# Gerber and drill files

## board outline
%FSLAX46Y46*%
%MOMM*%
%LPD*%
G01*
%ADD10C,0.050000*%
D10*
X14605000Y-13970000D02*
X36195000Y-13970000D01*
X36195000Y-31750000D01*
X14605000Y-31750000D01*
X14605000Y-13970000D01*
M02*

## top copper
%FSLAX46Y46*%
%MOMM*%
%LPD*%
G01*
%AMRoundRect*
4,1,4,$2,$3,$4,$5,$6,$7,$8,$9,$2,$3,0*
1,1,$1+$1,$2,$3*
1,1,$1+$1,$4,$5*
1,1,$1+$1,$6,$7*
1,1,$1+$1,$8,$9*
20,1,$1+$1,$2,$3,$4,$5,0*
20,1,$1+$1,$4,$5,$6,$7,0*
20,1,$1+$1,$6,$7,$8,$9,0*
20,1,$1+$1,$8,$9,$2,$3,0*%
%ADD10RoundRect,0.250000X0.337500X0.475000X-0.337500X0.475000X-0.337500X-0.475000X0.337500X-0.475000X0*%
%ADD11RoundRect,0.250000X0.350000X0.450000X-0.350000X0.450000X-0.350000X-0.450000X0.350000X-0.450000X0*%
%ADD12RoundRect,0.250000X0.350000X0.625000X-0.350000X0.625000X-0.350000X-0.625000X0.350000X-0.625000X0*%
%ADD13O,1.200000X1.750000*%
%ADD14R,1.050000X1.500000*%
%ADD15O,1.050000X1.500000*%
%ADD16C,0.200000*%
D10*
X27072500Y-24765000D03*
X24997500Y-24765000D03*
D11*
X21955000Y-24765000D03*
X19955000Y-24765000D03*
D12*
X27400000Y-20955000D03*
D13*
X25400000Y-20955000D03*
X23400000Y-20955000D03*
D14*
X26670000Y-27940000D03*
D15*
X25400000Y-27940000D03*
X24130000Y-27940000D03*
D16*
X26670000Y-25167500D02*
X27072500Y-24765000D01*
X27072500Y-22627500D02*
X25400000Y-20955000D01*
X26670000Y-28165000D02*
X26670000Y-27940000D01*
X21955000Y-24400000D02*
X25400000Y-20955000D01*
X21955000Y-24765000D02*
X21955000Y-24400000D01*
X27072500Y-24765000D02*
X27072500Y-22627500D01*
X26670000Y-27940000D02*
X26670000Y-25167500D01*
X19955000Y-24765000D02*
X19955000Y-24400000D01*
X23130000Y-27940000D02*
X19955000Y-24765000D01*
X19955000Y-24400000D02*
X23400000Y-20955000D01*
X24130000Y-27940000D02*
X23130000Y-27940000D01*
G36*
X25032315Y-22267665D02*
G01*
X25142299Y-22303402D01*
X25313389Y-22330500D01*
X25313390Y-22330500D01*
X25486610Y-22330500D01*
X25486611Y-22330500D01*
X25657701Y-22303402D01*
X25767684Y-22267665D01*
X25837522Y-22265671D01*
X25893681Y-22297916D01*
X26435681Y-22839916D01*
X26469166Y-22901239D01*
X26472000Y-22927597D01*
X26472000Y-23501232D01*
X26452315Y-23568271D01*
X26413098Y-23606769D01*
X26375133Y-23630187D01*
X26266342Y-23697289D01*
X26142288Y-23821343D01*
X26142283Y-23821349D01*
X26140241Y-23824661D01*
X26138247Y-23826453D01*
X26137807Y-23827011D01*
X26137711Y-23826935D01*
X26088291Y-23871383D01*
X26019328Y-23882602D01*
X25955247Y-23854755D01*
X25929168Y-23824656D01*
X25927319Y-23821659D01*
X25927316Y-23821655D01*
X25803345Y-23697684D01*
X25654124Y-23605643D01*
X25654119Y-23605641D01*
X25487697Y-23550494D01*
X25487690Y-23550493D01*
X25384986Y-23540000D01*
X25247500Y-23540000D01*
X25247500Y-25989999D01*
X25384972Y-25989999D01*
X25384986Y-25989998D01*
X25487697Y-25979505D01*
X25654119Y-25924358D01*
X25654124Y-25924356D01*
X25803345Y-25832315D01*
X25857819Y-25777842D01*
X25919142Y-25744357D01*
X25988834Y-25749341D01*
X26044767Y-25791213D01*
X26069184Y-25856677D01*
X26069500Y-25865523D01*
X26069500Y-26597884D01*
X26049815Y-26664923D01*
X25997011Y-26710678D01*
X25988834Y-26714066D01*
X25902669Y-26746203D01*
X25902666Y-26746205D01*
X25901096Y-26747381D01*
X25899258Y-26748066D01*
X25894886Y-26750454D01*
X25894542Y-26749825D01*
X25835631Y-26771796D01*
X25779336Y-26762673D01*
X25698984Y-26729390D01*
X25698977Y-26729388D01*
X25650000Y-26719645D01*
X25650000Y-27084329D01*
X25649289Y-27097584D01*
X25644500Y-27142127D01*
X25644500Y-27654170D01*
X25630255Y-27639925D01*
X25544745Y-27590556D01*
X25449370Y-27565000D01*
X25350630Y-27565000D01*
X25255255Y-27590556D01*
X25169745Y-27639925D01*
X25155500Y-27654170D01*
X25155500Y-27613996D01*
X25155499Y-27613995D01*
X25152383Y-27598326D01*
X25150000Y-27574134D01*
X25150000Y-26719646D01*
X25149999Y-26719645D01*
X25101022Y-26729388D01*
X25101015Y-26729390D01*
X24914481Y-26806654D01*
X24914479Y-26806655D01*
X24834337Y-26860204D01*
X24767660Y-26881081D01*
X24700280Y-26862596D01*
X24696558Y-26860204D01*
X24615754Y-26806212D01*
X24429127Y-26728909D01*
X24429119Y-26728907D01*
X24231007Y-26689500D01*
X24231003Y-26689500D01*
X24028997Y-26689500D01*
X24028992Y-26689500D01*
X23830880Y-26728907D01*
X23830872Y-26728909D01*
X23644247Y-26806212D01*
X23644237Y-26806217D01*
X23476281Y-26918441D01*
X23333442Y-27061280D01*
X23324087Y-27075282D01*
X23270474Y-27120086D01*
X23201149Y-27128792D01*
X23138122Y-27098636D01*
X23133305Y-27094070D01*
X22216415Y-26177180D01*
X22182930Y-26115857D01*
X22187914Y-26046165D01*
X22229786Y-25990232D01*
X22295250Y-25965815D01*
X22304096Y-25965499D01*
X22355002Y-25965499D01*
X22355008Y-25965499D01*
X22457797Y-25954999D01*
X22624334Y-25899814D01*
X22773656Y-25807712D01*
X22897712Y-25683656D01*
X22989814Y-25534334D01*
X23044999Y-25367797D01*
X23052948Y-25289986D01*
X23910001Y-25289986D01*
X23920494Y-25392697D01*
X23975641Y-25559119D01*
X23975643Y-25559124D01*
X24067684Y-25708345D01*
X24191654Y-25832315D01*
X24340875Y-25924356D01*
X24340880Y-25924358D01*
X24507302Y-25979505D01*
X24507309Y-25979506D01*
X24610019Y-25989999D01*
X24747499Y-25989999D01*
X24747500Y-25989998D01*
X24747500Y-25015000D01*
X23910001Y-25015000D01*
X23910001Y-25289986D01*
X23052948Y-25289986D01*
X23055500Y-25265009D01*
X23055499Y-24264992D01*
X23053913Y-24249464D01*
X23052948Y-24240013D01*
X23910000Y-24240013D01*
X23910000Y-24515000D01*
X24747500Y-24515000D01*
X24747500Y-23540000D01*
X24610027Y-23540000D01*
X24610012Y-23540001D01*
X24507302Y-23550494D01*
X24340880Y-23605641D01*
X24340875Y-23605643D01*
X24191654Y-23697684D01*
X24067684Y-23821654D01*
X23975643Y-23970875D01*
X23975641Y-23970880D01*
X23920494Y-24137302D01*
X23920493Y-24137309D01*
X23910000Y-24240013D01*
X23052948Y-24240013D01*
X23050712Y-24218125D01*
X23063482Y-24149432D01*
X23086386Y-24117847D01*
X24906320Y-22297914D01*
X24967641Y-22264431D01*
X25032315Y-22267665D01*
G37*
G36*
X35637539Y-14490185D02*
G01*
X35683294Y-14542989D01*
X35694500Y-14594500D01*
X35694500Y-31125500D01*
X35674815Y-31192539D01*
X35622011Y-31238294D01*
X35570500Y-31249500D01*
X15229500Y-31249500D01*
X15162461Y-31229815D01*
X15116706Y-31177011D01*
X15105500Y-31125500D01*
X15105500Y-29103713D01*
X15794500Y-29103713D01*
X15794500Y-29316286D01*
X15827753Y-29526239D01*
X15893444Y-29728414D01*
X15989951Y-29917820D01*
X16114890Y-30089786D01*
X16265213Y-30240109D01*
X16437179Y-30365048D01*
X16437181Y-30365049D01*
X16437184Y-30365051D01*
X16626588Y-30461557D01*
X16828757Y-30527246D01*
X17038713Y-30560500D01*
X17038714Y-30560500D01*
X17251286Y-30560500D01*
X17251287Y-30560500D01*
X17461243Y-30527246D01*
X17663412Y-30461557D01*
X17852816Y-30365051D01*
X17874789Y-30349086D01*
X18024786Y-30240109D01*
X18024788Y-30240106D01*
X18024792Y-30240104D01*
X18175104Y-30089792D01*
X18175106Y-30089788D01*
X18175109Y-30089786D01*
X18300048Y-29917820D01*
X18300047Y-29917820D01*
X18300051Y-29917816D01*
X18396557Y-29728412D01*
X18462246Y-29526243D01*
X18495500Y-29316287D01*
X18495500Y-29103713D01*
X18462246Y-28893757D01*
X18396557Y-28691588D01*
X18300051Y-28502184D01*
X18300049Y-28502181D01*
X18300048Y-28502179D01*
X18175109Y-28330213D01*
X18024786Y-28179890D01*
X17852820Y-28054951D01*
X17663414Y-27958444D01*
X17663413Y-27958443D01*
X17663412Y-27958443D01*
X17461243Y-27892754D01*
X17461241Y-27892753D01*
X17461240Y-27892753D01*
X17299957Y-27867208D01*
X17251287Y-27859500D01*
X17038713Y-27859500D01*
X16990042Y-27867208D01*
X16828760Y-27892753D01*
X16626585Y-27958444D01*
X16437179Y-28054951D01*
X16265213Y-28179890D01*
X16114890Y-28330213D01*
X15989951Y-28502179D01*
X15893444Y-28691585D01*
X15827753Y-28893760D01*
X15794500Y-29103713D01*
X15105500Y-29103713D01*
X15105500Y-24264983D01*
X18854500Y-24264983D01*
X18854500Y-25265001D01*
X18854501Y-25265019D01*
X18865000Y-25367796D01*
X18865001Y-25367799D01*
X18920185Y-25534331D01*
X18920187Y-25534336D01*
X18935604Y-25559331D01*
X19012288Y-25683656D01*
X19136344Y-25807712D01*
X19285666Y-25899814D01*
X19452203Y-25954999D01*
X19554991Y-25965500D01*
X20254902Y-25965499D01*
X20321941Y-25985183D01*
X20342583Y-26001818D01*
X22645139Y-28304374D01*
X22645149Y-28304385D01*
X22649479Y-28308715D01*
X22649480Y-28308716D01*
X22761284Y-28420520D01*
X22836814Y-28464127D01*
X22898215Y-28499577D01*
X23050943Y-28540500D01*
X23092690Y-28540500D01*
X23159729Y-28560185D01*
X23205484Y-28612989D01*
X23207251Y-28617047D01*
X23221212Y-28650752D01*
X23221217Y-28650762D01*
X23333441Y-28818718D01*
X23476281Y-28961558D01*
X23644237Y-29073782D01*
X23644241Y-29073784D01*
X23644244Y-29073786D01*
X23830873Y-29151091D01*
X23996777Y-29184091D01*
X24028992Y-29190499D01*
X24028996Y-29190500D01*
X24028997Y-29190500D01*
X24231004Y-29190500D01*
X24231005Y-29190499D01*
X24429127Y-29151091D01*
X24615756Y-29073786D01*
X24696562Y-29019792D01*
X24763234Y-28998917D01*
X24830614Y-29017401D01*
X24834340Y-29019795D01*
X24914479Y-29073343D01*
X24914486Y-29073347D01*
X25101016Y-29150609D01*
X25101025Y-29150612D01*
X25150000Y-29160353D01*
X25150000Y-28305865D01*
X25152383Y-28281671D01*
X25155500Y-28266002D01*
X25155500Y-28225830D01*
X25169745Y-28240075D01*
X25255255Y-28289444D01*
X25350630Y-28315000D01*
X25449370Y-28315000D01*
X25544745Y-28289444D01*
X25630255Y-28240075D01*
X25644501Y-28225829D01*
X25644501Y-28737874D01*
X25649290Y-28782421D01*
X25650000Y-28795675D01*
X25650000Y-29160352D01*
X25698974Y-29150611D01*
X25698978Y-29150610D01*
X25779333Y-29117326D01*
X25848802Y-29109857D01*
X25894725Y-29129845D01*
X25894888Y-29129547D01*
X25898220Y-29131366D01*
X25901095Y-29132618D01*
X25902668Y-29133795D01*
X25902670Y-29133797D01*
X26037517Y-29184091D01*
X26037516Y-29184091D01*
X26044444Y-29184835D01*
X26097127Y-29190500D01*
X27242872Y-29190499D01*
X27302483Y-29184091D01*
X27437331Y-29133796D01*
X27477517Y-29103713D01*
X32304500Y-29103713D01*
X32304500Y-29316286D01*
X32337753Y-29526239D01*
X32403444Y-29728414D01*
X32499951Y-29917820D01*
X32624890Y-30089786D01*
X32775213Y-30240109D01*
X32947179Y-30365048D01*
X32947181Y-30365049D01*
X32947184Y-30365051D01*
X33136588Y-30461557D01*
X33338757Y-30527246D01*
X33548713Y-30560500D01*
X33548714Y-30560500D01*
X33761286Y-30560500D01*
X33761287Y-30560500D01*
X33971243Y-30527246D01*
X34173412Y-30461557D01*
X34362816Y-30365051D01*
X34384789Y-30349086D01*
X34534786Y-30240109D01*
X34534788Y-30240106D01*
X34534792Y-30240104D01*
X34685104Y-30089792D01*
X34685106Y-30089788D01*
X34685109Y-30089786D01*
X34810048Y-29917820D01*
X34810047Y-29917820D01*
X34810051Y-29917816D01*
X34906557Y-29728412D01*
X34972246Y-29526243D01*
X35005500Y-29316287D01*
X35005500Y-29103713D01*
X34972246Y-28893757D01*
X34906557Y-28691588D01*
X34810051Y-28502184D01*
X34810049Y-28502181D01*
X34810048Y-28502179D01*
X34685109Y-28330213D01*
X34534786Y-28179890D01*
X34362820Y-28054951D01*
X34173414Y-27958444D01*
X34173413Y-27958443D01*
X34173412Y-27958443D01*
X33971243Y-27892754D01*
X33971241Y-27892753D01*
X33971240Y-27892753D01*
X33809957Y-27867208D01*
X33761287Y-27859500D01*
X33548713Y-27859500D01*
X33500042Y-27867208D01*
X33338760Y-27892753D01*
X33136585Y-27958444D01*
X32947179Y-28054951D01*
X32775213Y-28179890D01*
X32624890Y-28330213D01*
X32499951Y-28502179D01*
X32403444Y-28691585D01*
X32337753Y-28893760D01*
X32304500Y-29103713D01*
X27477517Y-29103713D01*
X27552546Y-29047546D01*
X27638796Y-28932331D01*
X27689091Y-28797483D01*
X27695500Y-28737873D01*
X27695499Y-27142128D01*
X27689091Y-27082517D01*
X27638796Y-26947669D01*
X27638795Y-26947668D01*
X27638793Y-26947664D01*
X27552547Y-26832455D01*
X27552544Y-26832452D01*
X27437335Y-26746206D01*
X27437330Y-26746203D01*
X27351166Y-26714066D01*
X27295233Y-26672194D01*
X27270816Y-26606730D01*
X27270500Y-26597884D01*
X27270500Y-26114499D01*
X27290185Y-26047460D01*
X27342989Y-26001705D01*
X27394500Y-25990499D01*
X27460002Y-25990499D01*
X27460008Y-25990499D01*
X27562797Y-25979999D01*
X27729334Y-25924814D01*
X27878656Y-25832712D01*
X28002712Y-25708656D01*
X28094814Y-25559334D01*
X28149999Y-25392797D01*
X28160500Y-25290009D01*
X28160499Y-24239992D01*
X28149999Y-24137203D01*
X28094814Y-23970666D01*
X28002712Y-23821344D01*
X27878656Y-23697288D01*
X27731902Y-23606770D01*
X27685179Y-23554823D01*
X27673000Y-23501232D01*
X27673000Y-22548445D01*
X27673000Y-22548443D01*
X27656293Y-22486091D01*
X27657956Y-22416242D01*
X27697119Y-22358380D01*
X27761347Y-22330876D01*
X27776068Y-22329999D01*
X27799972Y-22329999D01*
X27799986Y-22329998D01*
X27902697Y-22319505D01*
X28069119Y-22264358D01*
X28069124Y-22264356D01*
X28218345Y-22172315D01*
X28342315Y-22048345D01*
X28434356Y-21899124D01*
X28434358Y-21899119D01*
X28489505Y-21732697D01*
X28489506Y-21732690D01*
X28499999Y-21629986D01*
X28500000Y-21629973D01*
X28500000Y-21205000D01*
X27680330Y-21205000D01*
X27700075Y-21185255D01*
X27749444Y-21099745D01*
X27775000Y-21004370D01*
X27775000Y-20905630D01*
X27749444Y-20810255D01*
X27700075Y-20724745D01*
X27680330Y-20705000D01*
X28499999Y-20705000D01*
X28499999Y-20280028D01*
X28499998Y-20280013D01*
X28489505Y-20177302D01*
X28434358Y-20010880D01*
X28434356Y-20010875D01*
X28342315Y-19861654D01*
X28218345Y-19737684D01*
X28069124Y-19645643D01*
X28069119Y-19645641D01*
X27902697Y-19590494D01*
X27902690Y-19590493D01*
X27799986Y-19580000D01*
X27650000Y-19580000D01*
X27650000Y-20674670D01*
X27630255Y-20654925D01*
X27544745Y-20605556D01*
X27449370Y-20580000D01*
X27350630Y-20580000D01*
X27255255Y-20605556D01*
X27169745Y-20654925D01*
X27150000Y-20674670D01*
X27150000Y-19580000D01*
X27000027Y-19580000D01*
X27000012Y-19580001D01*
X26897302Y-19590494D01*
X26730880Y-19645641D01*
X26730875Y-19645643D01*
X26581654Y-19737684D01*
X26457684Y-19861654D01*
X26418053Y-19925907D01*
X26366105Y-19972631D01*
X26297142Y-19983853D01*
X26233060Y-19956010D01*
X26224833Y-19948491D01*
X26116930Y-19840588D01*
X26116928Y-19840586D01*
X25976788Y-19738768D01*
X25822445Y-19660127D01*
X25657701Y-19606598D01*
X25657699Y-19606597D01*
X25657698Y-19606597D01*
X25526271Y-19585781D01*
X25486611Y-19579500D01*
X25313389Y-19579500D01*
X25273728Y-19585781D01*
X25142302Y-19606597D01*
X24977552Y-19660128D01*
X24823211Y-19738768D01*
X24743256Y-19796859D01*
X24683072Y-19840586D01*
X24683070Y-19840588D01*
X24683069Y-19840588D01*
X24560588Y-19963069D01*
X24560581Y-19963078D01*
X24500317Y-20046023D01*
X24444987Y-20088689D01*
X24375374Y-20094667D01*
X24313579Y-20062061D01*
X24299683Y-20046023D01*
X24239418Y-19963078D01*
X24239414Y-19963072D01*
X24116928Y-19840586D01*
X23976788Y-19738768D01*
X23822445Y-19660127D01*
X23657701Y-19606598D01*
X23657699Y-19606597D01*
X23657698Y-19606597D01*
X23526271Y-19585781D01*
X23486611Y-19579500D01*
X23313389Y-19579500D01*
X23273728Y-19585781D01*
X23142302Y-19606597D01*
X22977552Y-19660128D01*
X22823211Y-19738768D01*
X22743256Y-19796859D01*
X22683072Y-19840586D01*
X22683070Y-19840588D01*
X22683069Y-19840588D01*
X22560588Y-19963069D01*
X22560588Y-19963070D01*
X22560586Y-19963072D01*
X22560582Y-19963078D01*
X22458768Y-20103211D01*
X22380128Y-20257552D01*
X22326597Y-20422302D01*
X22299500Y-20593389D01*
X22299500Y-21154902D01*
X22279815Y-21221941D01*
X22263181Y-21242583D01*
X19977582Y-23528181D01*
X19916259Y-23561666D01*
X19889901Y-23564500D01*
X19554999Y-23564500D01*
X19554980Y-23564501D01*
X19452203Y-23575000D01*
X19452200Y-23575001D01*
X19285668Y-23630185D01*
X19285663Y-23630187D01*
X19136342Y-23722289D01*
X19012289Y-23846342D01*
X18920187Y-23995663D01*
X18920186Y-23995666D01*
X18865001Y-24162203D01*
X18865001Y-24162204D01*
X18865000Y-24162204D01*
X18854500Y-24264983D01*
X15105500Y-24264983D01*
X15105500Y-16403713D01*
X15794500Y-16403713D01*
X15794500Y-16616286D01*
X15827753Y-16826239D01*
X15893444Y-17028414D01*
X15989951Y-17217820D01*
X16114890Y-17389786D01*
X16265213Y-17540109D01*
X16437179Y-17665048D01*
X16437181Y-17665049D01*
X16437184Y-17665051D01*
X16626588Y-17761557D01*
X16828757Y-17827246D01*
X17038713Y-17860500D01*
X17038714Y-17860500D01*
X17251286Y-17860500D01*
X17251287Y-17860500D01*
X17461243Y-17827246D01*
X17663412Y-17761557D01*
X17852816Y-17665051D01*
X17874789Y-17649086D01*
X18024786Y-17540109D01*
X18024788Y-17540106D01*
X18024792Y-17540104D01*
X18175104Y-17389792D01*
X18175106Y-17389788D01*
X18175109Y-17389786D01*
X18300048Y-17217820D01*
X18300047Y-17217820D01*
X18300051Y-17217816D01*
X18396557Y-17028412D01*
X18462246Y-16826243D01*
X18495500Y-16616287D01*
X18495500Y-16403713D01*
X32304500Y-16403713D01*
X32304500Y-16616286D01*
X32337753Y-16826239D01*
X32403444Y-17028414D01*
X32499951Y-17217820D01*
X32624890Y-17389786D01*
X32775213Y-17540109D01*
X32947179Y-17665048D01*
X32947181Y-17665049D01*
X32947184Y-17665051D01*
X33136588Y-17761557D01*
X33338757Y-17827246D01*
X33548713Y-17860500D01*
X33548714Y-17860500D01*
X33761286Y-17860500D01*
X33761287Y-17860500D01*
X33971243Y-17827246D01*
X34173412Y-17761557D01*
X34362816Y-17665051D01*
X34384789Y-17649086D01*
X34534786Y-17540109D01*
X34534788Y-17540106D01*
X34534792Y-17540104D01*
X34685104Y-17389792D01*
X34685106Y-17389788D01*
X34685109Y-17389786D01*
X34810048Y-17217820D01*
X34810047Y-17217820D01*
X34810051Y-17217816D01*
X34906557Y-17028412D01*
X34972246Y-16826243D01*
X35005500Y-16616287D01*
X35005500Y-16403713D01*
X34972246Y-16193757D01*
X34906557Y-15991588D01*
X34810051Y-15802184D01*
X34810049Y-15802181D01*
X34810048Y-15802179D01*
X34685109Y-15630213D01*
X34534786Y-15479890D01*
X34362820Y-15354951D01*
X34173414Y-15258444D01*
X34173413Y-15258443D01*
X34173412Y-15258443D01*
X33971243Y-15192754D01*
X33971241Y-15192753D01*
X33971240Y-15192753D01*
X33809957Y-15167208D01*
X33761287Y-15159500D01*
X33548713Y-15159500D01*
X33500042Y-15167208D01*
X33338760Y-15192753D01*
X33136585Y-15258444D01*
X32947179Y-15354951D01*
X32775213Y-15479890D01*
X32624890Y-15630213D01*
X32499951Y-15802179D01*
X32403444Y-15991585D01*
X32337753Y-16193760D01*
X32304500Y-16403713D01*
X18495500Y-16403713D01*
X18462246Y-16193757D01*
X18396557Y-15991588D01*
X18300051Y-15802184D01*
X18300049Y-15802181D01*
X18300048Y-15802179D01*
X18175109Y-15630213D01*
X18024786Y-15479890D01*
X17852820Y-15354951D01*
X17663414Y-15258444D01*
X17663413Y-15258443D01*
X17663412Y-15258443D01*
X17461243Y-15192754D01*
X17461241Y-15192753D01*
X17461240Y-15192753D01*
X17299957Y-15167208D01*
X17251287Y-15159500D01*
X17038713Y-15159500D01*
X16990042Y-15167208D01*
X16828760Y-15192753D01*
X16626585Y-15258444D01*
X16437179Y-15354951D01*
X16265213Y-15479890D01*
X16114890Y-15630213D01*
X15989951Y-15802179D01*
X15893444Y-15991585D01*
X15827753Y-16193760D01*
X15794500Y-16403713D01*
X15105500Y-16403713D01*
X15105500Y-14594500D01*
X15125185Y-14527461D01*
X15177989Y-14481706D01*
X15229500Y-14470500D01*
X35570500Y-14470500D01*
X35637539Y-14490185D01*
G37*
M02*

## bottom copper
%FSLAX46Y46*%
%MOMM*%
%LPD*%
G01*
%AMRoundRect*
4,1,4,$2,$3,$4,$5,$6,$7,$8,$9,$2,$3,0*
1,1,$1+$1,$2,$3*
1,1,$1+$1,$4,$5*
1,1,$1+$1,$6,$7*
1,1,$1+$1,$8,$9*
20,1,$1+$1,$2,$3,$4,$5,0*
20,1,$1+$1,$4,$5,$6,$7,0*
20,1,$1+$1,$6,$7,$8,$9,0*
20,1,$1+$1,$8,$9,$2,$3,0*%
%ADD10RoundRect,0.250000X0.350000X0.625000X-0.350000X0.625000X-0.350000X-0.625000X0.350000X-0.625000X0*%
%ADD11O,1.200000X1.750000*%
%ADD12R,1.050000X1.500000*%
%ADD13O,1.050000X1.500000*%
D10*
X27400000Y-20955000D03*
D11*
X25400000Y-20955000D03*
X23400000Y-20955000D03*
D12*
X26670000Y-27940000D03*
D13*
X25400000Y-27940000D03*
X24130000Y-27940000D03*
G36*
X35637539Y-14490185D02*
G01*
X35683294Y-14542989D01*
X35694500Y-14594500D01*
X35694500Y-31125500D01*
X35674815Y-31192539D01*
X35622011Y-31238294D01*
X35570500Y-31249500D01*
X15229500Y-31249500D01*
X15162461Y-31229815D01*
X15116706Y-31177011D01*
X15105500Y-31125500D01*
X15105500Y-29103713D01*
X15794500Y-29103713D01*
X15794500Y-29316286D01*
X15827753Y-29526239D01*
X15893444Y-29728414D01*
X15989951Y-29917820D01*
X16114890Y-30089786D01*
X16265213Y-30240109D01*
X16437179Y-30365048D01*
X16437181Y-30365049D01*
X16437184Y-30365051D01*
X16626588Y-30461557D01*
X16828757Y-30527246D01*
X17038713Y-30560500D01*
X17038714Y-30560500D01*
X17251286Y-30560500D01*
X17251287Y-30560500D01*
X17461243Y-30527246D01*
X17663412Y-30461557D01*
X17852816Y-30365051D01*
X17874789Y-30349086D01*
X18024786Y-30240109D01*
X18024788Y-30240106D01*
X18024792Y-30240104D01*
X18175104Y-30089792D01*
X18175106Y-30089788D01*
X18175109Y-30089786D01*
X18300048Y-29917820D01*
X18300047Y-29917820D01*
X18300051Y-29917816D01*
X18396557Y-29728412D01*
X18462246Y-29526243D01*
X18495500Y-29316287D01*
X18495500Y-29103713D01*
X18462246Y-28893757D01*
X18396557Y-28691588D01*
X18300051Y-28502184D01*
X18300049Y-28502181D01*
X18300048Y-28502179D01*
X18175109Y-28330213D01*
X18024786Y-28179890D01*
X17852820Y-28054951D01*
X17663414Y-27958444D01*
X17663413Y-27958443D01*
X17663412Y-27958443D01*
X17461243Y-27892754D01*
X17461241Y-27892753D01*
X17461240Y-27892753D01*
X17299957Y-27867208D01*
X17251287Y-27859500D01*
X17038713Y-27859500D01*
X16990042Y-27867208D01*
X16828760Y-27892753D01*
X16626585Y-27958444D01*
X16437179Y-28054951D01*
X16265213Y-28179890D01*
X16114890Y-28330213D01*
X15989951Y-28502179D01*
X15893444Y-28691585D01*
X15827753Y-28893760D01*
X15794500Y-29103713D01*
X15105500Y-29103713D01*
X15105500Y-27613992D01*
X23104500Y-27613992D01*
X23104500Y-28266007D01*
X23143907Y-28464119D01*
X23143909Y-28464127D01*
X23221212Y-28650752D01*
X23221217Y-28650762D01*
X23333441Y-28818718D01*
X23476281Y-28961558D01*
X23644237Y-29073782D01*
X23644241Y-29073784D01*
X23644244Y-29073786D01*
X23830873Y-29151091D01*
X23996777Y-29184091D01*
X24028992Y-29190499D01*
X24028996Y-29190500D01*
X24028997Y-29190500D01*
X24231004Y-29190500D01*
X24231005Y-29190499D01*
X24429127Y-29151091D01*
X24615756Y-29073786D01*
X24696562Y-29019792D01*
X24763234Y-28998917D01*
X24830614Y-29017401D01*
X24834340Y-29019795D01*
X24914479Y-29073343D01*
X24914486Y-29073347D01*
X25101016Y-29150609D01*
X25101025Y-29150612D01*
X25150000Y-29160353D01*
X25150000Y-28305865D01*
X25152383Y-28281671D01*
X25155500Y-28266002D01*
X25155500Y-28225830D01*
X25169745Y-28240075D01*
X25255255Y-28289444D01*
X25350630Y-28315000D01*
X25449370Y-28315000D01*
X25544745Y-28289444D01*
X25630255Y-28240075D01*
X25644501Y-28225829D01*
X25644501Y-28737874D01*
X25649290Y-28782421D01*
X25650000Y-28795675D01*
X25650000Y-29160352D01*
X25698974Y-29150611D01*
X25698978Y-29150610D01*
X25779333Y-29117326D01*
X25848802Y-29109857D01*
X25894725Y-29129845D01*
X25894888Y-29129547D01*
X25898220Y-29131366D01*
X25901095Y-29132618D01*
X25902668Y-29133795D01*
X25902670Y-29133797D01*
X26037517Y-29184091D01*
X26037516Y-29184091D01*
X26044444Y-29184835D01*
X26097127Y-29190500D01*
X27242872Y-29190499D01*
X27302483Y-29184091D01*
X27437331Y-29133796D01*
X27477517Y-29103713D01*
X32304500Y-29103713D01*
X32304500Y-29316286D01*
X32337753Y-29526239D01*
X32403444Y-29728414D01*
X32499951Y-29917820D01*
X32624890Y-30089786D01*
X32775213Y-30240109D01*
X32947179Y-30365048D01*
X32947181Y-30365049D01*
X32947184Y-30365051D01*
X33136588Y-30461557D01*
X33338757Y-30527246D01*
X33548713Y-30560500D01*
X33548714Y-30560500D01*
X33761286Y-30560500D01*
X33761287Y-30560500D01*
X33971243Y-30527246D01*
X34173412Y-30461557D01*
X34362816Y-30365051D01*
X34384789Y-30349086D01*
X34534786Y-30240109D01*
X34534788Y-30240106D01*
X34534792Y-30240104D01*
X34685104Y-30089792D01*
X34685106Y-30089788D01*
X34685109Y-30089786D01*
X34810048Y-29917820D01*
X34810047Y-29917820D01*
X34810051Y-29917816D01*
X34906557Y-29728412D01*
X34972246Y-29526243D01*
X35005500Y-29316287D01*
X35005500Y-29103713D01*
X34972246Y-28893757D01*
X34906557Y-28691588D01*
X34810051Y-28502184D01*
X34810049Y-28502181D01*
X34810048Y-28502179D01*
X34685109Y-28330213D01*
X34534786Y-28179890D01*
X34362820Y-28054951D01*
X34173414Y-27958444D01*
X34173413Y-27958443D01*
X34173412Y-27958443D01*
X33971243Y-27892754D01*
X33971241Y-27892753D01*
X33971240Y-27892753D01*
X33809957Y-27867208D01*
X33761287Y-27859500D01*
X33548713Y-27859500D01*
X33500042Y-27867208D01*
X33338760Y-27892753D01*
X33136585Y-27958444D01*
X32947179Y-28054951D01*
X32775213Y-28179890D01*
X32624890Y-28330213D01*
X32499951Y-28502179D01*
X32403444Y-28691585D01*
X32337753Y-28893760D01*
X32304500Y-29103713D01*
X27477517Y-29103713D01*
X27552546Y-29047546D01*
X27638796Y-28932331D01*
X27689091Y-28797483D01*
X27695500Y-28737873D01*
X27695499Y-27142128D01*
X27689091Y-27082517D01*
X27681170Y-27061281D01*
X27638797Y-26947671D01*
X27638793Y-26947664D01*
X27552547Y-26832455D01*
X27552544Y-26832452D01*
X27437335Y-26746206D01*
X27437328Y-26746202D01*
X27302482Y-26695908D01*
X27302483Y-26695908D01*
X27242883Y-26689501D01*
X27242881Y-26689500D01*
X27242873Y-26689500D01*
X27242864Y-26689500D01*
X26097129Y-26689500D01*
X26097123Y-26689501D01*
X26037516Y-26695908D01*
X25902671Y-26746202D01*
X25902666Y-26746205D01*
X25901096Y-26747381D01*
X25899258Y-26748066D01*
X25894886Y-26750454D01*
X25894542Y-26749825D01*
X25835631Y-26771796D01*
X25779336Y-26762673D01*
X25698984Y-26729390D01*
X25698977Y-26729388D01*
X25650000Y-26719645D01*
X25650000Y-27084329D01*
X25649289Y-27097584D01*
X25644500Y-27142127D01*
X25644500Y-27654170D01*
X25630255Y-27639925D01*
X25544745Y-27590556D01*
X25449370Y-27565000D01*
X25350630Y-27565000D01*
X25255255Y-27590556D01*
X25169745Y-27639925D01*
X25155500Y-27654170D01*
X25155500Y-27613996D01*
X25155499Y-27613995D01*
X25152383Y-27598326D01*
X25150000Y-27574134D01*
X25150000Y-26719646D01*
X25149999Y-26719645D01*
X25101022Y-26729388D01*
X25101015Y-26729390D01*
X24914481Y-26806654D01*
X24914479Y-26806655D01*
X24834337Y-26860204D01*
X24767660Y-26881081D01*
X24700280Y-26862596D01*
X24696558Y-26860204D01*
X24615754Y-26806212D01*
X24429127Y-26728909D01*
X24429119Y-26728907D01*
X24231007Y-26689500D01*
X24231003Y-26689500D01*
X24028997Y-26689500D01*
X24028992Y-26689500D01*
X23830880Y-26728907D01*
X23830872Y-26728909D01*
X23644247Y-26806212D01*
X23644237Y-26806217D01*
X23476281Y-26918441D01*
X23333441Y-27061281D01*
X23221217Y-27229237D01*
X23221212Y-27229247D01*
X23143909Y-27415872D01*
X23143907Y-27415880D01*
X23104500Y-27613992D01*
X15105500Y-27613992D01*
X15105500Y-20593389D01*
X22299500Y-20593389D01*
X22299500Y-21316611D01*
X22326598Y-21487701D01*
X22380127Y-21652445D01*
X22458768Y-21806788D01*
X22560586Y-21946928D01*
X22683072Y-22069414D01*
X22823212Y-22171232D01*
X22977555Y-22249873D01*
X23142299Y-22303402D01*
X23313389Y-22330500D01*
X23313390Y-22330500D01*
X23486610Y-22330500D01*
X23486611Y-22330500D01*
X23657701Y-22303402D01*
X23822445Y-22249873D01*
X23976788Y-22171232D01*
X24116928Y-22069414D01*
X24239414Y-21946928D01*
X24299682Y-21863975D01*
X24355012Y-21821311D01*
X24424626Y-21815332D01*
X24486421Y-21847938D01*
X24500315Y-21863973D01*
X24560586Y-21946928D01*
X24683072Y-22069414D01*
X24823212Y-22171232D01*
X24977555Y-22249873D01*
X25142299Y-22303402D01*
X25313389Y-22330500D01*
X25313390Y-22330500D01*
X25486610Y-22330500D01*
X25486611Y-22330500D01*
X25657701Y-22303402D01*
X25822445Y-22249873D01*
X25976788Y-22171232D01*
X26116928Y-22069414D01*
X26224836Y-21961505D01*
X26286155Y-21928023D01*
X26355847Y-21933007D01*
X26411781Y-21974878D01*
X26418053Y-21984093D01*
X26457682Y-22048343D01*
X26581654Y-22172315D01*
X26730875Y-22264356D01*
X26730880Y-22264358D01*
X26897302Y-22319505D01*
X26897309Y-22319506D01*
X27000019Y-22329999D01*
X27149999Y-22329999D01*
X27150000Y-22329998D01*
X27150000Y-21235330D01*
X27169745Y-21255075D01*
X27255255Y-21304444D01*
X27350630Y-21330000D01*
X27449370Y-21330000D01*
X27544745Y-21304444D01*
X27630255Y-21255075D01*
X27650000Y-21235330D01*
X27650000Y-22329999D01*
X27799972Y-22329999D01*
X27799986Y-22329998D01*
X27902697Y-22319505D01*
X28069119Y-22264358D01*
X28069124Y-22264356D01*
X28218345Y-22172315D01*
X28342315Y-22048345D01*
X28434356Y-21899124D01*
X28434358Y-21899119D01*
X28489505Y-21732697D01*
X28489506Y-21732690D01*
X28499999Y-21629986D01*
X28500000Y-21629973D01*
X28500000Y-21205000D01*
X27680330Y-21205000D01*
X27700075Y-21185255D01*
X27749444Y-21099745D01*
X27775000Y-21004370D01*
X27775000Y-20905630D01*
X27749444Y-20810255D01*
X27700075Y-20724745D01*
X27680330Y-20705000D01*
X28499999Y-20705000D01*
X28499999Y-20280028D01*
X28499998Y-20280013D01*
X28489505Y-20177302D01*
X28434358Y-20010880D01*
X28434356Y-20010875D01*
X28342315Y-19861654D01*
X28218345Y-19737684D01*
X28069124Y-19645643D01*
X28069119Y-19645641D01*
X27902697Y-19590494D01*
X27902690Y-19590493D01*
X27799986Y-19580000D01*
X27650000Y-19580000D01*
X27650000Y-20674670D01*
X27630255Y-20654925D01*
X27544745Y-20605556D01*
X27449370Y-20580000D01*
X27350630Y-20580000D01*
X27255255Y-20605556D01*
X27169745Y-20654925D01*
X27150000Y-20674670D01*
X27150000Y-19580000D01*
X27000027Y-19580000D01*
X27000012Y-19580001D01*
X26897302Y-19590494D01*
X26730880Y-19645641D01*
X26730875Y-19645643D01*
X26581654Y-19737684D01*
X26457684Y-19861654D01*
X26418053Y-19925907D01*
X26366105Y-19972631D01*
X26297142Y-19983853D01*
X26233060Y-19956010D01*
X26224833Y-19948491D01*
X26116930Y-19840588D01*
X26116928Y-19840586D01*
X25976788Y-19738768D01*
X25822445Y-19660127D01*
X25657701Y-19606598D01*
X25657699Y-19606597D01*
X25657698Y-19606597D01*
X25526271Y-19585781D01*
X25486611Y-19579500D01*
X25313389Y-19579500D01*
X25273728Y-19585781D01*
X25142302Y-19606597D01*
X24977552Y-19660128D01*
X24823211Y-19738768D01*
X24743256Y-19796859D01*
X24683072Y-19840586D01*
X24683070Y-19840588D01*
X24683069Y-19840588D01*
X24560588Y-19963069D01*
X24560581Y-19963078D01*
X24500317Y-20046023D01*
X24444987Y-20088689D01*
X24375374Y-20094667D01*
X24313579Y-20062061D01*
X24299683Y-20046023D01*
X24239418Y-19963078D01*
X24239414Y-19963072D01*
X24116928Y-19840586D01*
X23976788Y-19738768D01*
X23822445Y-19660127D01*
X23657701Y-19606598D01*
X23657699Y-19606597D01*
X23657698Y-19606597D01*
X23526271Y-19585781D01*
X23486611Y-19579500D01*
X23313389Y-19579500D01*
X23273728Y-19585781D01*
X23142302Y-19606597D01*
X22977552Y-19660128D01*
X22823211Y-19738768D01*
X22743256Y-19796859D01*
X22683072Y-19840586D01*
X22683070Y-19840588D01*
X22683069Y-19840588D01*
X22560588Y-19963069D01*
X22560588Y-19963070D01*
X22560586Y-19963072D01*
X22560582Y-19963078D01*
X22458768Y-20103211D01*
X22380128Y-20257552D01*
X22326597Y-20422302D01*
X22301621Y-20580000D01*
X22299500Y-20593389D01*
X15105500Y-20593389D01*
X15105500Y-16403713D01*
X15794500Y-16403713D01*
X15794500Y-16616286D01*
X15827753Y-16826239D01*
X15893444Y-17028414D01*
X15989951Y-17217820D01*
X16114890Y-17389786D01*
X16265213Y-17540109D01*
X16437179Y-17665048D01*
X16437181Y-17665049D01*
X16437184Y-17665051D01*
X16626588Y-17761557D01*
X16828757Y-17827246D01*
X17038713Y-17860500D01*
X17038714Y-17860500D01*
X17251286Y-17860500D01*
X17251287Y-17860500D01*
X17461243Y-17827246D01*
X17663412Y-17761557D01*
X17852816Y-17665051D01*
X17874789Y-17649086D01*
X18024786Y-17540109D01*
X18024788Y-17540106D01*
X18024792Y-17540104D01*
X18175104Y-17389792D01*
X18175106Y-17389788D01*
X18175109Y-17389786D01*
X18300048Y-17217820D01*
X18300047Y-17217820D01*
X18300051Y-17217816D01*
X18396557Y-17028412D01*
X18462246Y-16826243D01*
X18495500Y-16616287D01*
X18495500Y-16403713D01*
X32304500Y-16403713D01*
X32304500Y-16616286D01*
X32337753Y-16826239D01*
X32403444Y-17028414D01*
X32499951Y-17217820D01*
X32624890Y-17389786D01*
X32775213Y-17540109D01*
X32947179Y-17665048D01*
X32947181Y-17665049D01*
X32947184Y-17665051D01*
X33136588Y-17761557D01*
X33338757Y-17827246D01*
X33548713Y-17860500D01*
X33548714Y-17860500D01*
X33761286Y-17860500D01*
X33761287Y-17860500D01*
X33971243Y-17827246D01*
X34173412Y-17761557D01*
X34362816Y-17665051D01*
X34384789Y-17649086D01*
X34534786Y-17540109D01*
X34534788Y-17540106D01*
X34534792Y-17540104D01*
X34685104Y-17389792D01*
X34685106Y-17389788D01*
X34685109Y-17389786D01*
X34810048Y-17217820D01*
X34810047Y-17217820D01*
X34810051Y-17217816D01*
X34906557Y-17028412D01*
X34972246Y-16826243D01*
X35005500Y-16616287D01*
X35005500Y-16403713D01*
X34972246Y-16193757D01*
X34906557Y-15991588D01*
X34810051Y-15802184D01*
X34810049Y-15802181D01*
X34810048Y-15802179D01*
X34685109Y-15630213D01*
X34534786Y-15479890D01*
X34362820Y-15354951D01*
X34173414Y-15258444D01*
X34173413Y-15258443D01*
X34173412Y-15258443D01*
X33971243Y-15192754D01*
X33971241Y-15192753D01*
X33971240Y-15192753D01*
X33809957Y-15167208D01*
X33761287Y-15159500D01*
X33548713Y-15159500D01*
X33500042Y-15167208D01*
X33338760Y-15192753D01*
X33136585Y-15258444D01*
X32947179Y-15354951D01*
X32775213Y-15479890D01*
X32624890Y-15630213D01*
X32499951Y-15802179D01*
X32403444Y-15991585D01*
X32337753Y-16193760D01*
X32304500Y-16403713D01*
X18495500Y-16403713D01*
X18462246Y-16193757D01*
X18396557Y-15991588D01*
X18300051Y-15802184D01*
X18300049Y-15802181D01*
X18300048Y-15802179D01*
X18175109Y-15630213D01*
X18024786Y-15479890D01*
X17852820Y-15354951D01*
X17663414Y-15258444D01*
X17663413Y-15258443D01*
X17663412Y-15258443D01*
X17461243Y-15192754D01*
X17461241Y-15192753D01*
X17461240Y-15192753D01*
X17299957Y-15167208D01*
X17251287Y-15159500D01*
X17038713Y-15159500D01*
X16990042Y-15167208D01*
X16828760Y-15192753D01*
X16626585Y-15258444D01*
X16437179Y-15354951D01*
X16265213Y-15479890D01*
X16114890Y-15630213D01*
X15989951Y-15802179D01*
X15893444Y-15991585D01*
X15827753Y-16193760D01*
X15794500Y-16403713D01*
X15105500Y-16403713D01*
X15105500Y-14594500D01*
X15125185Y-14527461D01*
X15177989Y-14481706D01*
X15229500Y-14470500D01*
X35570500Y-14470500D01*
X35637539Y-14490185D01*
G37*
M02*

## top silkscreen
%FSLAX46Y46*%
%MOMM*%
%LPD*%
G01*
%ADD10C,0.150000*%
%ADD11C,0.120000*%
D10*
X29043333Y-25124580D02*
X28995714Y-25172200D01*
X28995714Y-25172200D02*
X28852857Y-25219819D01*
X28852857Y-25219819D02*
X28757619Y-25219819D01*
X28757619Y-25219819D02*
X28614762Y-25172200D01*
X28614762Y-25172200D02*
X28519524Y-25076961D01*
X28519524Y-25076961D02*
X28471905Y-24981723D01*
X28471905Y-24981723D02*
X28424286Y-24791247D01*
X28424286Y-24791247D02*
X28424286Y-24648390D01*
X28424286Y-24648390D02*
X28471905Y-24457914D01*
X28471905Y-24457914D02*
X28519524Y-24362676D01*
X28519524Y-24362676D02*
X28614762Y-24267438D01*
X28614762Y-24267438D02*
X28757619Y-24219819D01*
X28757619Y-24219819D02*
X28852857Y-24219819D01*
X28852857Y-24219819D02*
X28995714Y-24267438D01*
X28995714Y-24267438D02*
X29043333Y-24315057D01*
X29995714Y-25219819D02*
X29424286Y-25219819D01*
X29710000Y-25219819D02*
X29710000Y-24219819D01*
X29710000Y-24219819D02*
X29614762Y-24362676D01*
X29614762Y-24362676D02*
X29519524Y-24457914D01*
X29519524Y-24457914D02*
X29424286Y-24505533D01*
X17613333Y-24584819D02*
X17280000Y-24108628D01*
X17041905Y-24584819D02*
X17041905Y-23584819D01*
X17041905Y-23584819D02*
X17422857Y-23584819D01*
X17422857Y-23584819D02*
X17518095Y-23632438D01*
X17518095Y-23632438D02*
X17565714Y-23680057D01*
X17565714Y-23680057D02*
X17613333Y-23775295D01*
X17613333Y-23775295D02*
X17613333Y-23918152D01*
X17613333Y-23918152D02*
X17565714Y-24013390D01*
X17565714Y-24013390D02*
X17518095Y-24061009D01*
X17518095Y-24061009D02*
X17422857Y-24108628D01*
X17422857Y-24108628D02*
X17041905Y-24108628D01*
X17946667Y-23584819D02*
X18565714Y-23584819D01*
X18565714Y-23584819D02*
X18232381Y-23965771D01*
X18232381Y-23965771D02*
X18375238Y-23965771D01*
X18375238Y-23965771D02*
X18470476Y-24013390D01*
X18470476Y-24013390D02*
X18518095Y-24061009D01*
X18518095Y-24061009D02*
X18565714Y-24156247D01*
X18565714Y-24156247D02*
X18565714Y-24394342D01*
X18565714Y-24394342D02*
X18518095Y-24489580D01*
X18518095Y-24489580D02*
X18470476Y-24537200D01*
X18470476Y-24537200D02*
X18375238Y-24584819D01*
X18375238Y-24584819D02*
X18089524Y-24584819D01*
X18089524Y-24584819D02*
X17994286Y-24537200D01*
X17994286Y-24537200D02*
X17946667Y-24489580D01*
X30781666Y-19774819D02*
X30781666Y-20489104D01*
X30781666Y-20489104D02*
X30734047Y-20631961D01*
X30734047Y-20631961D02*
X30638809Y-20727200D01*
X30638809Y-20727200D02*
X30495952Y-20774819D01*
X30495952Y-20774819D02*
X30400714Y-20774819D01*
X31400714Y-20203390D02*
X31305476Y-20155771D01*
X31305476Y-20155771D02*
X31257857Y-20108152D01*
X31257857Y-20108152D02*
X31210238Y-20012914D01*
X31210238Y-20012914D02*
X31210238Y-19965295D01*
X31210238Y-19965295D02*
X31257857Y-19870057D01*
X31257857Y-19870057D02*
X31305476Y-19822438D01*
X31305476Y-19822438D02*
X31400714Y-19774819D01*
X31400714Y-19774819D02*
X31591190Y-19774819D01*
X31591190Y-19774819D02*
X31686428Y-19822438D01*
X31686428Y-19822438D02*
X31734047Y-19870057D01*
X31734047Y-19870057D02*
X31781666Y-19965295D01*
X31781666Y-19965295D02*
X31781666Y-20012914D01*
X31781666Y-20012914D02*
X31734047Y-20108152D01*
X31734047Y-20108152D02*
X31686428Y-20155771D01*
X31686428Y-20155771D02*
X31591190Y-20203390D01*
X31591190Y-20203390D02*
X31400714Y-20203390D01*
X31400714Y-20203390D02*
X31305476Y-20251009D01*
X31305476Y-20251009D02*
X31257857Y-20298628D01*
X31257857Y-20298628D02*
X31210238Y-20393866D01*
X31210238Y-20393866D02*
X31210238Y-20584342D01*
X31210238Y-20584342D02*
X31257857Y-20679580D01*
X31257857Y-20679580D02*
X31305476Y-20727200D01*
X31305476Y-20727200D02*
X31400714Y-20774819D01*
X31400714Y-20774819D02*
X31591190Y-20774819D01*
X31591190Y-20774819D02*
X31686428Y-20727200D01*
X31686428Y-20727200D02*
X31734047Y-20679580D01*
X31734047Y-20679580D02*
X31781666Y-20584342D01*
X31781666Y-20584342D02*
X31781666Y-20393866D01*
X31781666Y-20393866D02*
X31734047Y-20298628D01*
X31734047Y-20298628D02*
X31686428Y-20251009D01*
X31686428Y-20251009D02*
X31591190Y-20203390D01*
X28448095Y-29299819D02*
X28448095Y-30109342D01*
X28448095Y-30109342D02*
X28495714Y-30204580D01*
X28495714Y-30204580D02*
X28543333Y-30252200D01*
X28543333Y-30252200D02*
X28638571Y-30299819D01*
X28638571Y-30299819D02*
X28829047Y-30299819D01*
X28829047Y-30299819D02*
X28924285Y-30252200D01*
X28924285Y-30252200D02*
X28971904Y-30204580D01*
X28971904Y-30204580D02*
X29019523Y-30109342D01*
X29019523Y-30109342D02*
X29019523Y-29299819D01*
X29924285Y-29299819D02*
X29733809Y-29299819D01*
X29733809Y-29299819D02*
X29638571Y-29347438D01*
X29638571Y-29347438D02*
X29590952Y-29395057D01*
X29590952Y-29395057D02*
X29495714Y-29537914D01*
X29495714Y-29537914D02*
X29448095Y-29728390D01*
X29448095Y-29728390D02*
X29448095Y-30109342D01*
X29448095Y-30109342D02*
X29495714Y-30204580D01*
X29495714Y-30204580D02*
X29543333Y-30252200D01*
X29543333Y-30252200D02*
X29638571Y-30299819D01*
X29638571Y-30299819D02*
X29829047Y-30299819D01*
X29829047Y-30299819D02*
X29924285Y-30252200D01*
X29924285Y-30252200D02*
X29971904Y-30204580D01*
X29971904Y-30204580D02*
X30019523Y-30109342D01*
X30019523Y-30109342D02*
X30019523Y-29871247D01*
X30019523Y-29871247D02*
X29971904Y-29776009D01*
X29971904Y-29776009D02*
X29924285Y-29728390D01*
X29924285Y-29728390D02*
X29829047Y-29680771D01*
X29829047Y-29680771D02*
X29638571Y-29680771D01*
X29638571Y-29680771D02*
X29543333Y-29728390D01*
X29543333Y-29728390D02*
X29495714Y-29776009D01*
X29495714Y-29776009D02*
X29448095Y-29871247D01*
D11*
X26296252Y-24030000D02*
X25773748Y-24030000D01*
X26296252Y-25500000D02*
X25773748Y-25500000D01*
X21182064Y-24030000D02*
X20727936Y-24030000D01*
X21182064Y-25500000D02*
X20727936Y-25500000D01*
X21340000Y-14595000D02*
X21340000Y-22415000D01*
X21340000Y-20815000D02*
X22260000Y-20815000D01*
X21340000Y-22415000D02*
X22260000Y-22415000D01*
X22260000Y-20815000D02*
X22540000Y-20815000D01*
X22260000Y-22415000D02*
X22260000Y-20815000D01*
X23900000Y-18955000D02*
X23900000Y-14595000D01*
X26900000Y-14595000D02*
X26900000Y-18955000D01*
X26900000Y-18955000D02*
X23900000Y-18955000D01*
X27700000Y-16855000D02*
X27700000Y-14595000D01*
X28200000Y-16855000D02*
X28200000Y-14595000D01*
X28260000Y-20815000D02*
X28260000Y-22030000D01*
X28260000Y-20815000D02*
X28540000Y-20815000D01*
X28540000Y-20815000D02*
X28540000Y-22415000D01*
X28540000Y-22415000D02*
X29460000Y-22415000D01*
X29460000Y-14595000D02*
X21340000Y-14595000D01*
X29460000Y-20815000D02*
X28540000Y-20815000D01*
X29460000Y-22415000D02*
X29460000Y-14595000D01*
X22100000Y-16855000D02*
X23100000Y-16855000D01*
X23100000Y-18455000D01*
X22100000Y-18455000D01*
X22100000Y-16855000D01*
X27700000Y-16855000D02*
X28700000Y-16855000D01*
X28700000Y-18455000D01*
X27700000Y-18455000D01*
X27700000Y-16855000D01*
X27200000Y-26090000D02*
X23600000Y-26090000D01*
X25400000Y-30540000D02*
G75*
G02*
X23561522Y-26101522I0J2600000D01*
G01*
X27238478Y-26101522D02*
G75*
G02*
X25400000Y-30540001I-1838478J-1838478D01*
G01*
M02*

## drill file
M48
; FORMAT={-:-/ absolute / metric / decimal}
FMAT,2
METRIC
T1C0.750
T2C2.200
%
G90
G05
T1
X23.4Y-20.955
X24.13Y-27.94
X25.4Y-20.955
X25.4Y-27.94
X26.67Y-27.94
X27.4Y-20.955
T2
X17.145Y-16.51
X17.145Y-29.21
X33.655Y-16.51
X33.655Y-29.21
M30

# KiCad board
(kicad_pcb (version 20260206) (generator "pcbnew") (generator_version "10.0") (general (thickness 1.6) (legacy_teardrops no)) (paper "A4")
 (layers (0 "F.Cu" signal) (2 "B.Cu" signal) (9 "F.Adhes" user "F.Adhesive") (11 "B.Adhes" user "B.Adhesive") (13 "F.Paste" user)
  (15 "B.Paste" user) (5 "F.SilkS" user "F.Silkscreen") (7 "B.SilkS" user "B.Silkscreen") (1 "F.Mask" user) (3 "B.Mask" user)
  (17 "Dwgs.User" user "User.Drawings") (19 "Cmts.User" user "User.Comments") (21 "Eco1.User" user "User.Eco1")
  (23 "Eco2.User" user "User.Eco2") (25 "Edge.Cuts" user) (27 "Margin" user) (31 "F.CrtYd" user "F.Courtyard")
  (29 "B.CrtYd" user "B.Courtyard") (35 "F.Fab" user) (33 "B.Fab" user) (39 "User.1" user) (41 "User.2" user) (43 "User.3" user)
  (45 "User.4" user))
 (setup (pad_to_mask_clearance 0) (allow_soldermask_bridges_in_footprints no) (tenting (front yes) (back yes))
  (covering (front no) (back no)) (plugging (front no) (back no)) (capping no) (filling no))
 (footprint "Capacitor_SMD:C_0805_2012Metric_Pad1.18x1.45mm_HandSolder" (layer "F.Cu") (at 26.035 24.765 180)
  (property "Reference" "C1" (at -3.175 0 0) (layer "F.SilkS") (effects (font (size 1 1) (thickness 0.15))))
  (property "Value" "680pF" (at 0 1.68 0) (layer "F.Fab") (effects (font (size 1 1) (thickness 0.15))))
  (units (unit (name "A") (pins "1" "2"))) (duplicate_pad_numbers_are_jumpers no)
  (fp_line (start -0.261252 0.735) (end 0.261252 0.735) (stroke (width 0.12) (type solid)) (layer "F.SilkS"))
  (fp_line (start -0.261252 -0.735) (end 0.261252 -0.735) (stroke (width 0.12) (type solid)) (layer "F.SilkS"))
  (pad "1" smd roundrect (at -1.0375 0 180) (size 1.175 1.45) (layers "F.Cu" "F.Mask" "F.Paste") (roundrect_rratio 0.212766) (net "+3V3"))
  (pad "2" smd roundrect (at 1.0375 0 180) (size 1.175 1.45) (layers "F.Cu" "F.Mask" "F.Paste") (roundrect_rratio 0.212766) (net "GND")))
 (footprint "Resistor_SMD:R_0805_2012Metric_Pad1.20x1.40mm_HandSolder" (layer "F.Cu") (at 20.955 24.765 180)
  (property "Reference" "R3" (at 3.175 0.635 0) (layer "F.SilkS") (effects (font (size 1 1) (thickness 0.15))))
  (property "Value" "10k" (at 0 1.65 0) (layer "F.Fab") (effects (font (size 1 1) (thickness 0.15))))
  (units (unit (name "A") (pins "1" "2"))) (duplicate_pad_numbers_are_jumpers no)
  (fp_line (start -0.227064 0.735) (end 0.227064 0.735) (stroke (width 0.12) (type solid)) (layer "F.SilkS"))
  (fp_line (start -0.227064 -0.735) (end 0.227064 -0.735) (stroke (width 0.12) (type solid)) (layer "F.SilkS"))
  (pad "1" smd roundrect (at -1 0 180) (size 1.2 1.4) (layers "F.Cu" "F.Mask" "F.Paste") (roundrect_rratio 0.208333) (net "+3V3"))
  (pad "2" smd roundrect (at 1 0 180) (size 1.2 1.4) (layers "F.Cu" "F.Mask" "F.Paste") (roundrect_rratio 0.208333) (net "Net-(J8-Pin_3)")))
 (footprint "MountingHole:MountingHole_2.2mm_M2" (layer "F.Cu") (at 17.145 29.21)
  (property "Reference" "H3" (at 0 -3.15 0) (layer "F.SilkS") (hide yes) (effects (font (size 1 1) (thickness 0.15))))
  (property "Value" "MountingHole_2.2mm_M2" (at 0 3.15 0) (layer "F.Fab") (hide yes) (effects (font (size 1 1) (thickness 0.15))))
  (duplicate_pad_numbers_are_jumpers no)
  (pad "" np_thru_hole circle (at 0 0) (size 2.2 2.2) (drill 2.2) (layers "*.Cu" "*.Mask")))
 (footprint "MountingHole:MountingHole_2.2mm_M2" (layer "F.Cu") (at 17.145 16.51)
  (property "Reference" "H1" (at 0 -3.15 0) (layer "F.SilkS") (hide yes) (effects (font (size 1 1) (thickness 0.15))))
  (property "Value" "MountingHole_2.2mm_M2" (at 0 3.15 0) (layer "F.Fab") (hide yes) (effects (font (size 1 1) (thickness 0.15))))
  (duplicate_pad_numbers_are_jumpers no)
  (pad "" np_thru_hole circle (at 0 0) (size 2.2 2.2) (drill 2.2) (layers "*.Cu" "*.Mask")))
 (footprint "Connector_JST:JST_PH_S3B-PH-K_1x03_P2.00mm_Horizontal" (layer "F.Cu") (at 27.4 20.955 180)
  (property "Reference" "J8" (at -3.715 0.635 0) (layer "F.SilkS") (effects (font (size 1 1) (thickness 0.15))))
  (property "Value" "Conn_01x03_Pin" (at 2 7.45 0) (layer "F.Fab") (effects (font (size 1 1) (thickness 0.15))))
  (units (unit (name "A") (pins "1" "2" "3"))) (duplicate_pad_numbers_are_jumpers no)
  (fp_line (start 6.06 6.36) (end 6.06 -1.46) (stroke (width 0.12) (type solid)) (layer "F.SilkS"))
  (fp_line (start 6.06 0.14) (end 5.14 0.14) (stroke (width 0.12) (type solid)) (layer "F.SilkS"))
  (fp_line (start 6.06 -1.46) (end 5.14 -1.46) (stroke (width 0.12) (type solid)) (layer "F.SilkS"))
  (fp_line (start 5.14 0.14) (end 4.86 0.14) (stroke (width 0.12) (type solid)) (layer "F.SilkS"))
  (fp_line (start 5.14 -1.46) (end 5.14 0.14) (stroke (width 0.12) (type solid)) (layer "F.SilkS"))
  (fp_line (start 3.5 2) (end 3.5 6.36) (stroke (width 0.12) (type solid)) (layer "F.SilkS"))
  (fp_line (start 0.5 6.36) (end 0.5 2) (stroke (width 0.12) (type solid)) (layer "F.SilkS"))
  (fp_line (start 0.5 2) (end 3.5 2) (stroke (width 0.12) (type solid)) (layer "F.SilkS"))
  (fp_line (start -0.3 4.1) (end -0.3 6.36) (stroke (width 0.12) (type solid)) (layer "F.SilkS"))
  (fp_line (start -0.8 4.1) (end -0.8 6.36) (stroke (width 0.12) (type solid)) (layer "F.SilkS"))
  (fp_line (start -0.86 0.14) (end -0.86 -1.075) (stroke (width 0.12) (type solid)) (layer "F.SilkS"))
  (fp_line (start -0.86 0.14) (end -1.14 0.14) (stroke (width 0.12) (type solid)) (layer "F.SilkS"))
  (fp_line (start -1.14 0.14) (end -1.14 -1.46) (stroke (width 0.12) (type solid)) (layer "F.SilkS"))
  (fp_line (start -1.14 -1.46) (end -2.06 -1.46) (stroke (width 0.12) (type solid)) (layer "F.SilkS"))
  (fp_line (start -2.06 6.36) (end 6.06 6.36) (stroke (width 0.12) (type solid)) (layer "F.SilkS"))
  (fp_line (start -2.06 0.14) (end -1.14 0.14) (stroke (width 0.12) (type solid)) (layer "F.SilkS"))
  (fp_line (start -2.06 -1.46) (end -2.06 6.36) (stroke (width 0.12) (type solid)) (layer "F.SilkS"))
  (fp_rect (start 4.3 2.5) (end 5.3 4.1) (stroke (width 0.12) (type solid)) (fill no) (layer "F.SilkS"))
  (fp_rect (start -1.3 2.5) (end -0.3 4.1) (stroke (width 0.12) (type solid)) (fill no) (layer "F.SilkS"))
  (pad "1" thru_hole roundrect (at 0 0 180) (size 1.2 1.75) (drill 0.75) (layers "*.Cu" "*.Mask") (remove_unused_layers no)
   (roundrect_rratio 0.208333) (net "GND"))
  (pad "2" thru_hole oval (at 2 0 180) (size 1.2 1.75) (drill 0.75) (layers "*.Cu" "*.Mask") (remove_unused_layers no) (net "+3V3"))
  (pad "3" thru_hole oval (at 4 0 180) (size 1.2 1.75) (drill 0.75) (layers "*.Cu" "*.Mask") (remove_unused_layers no)
   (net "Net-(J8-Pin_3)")))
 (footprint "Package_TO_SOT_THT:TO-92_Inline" (layer "F.Cu") (at 26.67 27.94 180)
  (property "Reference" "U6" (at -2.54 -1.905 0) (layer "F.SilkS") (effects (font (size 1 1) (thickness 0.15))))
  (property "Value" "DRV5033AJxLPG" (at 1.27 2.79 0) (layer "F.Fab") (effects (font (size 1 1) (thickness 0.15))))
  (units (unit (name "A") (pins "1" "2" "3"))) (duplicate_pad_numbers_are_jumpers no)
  (fp_line (start -0.53 1.85) (end 3.07 1.85) (stroke (width 0.12) (type solid)) (layer "F.SilkS"))
  (fp_arc (start 1.27 -2.6) (mid 3.672087 -0.994977) (end 3.108478 1.838478) (stroke (width 0.12) (type solid)) (layer "F.SilkS"))
  (fp_arc (start -0.568478 1.838478) (mid -1.132087 -0.994977) (end 1.27 -2.6) (stroke (width 0.12) (type solid)) (layer "F.SilkS"))
  (pad "1" thru_hole rect (at 0 0 180) (size 1.05 1.5) (drill 0.75) (layers "*.Cu" "*.Mask") (remove_unused_layers no) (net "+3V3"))
  (pad "2" thru_hole oval (at 1.27 0 180) (size 1.05 1.5) (drill 0.75) (layers "*.Cu" "*.Mask") (remove_unused_layers no) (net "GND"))
  (pad "3" thru_hole oval (at 2.54 0 180) (size 1.05 1.5) (drill 0.75) (layers "*.Cu" "*.Mask") (remove_unused_layers no)
   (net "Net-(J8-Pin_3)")))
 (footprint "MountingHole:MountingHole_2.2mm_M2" (layer "F.Cu") (at 33.655 16.51)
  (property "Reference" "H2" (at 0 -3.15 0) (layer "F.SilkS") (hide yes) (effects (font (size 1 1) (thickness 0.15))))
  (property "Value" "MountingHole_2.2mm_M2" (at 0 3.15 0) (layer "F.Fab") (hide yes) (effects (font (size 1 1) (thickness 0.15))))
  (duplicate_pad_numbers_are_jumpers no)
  (pad "" np_thru_hole circle (at 0 0) (size 2.2 2.2) (drill 2.2) (layers "*.Cu" "*.Mask")))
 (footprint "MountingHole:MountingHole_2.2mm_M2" (layer "F.Cu") (at 33.655 29.21)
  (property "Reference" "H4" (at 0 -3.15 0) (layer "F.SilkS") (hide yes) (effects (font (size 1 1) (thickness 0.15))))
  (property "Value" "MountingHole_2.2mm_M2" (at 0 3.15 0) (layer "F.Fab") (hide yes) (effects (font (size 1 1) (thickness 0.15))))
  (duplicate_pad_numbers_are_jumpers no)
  (pad "" np_thru_hole circle (at 0 0) (size 2.2 2.2) (drill 2.2) (layers "*.Cu" "*.Mask")))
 (gr_rect (start 14.605 13.97) (end 36.195 31.75) (stroke (width 0.05) (type solid)) (fill no) (layer "Edge.Cuts"))
 (segment (start 26.67 25.1675) (end 27.0725 24.765) (width 0.2) (layer "F.Cu") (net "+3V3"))
 (segment (start 27.0725 22.6275) (end 25.4 20.955) (width 0.2) (layer "F.Cu") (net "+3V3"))
 (segment (start 26.67 28.165) (end 26.67 27.94) (width 0.2) (layer "F.Cu") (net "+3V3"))
 (segment (start 21.955 24.4) (end 25.4 20.955) (width 0.2) (layer "F.Cu") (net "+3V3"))
 (segment (start 21.955 24.765) (end 21.955 24.4) (width 0.2) (layer "F.Cu") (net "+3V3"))
 (segment (start 27.0725 24.765) (end 27.0725 22.6275) (width 0.2) (layer "F.Cu") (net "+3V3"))
 (segment (start 26.67 27.94) (end 26.67 25.1675) (width 0.2) (layer "F.Cu") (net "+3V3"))
 (segment (start 19.955 24.765) (end 19.955 24.4) (width 0.2) (layer "F.Cu") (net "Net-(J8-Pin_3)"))
 (segment (start 23.13 27.94) (end 19.955 24.765) (width 0.2) (layer "F.Cu") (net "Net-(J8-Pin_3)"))
 (segment (start 19.955 24.4) (end 23.4 20.955) (width 0.2) (layer "F.Cu") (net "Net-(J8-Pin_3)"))
 (segment (start 24.13 27.94) (end 23.13 27.94) (width 0.2) (layer "F.Cu") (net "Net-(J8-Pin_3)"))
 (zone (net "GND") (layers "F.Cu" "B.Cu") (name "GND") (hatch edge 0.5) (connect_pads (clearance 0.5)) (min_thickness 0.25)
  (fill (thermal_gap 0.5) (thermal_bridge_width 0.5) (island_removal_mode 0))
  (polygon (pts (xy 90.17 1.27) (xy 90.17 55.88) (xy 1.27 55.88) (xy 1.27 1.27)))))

